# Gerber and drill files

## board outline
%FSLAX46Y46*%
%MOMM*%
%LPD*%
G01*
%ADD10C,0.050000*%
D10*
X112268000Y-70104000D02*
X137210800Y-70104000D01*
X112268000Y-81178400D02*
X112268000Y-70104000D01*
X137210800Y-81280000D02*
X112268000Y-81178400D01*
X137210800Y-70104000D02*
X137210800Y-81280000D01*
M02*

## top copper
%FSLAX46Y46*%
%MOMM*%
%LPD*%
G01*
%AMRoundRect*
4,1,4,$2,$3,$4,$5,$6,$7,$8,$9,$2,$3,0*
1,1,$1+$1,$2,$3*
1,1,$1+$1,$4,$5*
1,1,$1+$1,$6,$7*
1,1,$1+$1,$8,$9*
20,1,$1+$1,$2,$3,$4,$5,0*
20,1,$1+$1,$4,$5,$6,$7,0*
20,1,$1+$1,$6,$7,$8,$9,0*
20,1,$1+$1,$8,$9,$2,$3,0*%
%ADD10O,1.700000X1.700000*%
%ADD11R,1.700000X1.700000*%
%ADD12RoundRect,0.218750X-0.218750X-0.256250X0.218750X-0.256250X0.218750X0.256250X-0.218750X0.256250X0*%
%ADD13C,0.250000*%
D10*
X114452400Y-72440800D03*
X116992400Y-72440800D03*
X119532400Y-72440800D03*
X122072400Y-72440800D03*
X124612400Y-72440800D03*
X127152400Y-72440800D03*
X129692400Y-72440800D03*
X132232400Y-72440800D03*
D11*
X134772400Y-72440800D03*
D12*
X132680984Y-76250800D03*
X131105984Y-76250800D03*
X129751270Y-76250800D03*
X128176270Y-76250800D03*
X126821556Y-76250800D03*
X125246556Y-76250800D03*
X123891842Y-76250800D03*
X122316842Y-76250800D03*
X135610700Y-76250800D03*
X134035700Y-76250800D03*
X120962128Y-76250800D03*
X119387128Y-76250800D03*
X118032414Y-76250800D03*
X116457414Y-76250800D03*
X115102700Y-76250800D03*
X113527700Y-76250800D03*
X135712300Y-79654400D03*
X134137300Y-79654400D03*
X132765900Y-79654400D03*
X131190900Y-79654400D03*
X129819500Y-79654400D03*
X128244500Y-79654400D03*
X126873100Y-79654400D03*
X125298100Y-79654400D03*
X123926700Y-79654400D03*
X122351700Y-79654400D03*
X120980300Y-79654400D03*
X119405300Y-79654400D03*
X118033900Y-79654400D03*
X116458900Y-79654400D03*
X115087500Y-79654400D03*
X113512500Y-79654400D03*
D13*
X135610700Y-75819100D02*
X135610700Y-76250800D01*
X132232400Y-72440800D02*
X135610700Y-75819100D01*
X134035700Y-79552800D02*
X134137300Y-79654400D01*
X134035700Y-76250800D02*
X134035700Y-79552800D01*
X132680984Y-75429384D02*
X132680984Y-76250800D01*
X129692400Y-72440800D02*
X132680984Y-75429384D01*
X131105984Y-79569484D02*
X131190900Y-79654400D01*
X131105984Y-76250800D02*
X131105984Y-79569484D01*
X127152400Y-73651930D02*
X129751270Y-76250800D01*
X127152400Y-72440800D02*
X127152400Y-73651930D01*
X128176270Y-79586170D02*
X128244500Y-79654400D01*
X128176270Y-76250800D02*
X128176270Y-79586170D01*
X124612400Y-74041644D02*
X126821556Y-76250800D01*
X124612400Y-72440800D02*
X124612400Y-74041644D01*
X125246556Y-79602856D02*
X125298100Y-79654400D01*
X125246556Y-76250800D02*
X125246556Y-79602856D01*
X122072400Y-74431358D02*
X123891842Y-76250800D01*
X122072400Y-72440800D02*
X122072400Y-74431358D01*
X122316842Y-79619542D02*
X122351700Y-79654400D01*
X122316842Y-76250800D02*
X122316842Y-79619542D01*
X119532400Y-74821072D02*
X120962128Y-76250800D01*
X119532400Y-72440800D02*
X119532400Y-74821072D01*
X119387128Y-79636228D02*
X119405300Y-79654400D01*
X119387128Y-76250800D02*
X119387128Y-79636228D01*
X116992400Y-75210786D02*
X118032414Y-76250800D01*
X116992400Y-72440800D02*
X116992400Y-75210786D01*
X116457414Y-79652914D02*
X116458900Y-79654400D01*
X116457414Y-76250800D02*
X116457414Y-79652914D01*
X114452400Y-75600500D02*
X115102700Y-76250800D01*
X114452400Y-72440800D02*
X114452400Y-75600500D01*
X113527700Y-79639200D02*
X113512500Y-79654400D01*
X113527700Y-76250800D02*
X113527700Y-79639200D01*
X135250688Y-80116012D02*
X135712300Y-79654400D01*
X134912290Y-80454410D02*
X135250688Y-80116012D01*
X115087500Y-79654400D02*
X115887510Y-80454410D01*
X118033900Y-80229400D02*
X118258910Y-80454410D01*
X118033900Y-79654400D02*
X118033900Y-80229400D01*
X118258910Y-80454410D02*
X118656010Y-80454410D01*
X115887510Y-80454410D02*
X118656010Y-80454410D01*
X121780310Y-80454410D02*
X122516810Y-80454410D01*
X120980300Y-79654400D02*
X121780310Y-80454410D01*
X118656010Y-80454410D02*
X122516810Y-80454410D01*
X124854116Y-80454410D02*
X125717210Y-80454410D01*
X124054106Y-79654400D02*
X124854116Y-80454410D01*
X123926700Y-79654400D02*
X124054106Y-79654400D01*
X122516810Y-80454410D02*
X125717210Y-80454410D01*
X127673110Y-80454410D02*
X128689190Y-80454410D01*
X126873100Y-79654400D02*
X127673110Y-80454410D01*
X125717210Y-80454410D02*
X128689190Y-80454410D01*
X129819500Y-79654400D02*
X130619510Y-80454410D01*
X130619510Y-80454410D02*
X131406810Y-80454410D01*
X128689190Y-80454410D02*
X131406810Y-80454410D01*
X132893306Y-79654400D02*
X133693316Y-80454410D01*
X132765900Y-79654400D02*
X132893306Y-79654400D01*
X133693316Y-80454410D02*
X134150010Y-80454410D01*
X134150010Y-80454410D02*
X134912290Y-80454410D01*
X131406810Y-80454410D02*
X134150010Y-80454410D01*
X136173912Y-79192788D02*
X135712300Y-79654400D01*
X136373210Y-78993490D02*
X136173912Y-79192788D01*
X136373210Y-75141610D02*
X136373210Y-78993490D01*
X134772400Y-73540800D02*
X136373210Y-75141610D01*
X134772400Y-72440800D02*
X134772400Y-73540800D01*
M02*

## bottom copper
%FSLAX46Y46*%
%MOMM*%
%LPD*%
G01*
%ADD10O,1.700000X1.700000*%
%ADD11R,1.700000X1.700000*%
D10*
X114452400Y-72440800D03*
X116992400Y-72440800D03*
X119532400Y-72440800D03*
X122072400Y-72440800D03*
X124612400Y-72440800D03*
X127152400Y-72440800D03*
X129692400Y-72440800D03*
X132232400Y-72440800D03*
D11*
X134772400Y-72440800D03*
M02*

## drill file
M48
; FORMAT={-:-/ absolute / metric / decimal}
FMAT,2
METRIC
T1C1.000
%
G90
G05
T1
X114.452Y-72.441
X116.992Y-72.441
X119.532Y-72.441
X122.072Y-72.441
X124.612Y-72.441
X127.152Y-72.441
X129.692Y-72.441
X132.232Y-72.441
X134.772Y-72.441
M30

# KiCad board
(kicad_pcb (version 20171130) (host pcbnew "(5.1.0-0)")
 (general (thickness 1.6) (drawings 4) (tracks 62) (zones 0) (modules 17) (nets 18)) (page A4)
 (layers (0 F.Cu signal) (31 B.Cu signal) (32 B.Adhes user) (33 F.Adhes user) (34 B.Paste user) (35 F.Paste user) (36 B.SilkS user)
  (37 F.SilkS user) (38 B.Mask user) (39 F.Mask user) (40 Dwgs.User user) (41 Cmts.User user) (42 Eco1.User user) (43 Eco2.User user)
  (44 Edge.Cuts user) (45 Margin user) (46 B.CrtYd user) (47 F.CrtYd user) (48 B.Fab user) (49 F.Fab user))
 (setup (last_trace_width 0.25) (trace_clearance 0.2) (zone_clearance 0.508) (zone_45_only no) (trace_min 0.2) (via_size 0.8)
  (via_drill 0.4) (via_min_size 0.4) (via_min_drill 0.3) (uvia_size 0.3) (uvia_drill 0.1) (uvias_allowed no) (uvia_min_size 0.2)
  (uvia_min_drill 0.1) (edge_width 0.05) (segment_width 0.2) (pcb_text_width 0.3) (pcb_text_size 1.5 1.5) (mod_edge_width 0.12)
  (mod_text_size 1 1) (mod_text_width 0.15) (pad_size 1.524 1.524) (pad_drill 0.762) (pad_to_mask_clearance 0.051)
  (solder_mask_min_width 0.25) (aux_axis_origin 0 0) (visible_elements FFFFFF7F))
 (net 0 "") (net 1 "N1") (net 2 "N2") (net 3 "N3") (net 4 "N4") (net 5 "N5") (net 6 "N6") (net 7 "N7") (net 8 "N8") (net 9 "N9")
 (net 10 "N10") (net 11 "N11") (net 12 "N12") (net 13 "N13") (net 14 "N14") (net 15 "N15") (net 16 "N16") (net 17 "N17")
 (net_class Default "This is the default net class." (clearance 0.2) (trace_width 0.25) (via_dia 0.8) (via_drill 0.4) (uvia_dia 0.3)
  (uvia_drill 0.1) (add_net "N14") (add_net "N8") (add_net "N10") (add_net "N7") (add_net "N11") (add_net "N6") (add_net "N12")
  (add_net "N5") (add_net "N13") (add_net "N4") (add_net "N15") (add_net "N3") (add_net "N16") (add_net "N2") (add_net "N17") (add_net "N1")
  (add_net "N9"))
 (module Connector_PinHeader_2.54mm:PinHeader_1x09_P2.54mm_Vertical (layer B.Cu) (at 134.7724 72.4408 90)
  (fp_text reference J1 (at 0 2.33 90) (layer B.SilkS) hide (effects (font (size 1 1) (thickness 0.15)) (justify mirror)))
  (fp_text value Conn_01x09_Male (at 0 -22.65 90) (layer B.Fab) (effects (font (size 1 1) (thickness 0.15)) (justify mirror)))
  (pad 9 thru_hole oval (at 0 -20.32 90) (size 1.7 1.7) (drill 1) (layers *.Cu *.Mask) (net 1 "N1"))
  (pad 8 thru_hole oval (at 0 -17.78 90) (size 1.7 1.7) (drill 1) (layers *.Cu *.Mask) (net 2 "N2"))
  (pad 7 thru_hole oval (at 0 -15.24 90) (size 1.7 1.7) (drill 1) (layers *.Cu *.Mask) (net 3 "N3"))
  (pad 6 thru_hole oval (at 0 -12.7 90) (size 1.7 1.7) (drill 1) (layers *.Cu *.Mask) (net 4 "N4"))
  (pad 5 thru_hole oval (at 0 -10.16 90) (size 1.7 1.7) (drill 1) (layers *.Cu *.Mask) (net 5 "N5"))
  (pad 4 thru_hole oval (at 0 -7.62 90) (size 1.7 1.7) (drill 1) (layers *.Cu *.Mask) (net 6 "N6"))
  (pad 3 thru_hole oval (at 0 -5.08 90) (size 1.7 1.7) (drill 1) (layers *.Cu *.Mask) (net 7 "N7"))
  (pad 2 thru_hole oval (at 0 -2.54 90) (size 1.7 1.7) (drill 1) (layers *.Cu *.Mask) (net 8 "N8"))
  (pad 1 thru_hole rect (at 0 0 90) (size 1.7 1.7) (drill 1) (layers *.Cu *.Mask) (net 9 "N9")))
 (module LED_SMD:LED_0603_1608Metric (layer F.Cu) (at 131.893484 76.2508)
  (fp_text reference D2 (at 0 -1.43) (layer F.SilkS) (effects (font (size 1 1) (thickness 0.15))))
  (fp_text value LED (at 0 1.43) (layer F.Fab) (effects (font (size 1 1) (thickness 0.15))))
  (pad 2 smd roundrect (at 0.7875 0) (size 0.875 0.95) (layers F.Cu F.Paste F.Mask) (roundrect_rratio 0.25) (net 7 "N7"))
  (pad 1 smd roundrect (at -0.7875 0) (size 0.875 0.95) (layers F.Cu F.Paste F.Mask) (roundrect_rratio 0.25) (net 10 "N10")))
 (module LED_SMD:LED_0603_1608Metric (layer F.Cu) (at 128.96377 76.2508)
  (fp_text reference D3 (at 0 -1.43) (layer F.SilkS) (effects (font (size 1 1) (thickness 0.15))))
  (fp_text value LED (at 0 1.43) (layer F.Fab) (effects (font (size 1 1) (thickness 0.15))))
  (pad 2 smd roundrect (at 0.7875 0) (size 0.875 0.95) (layers F.Cu F.Paste F.Mask) (roundrect_rratio 0.25) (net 6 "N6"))
  (pad 1 smd roundrect (at -0.7875 0) (size 0.875 0.95) (layers F.Cu F.Paste F.Mask) (roundrect_rratio 0.25) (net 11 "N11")))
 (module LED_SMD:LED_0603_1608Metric (layer F.Cu) (at 126.034056 76.2508)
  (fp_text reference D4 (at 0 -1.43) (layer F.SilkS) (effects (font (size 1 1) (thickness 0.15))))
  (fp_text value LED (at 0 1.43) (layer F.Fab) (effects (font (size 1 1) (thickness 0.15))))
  (pad 2 smd roundrect (at 0.7875 0) (size 0.875 0.95) (layers F.Cu F.Paste F.Mask) (roundrect_rratio 0.25) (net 5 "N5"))
  (pad 1 smd roundrect (at -0.7875 0) (size 0.875 0.95) (layers F.Cu F.Paste F.Mask) (roundrect_rratio 0.25) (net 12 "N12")))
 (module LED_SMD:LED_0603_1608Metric (layer F.Cu) (at 123.104342 76.2508)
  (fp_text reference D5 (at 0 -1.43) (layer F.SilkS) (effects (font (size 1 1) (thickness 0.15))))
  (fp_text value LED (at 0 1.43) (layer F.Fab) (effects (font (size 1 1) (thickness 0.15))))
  (pad 2 smd roundrect (at 0.7875 0) (size 0.875 0.95) (layers F.Cu F.Paste F.Mask) (roundrect_rratio 0.25) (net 4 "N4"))
  (pad 1 smd roundrect (at -0.7875 0) (size 0.875 0.95) (layers F.Cu F.Paste F.Mask) (roundrect_rratio 0.25) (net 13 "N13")))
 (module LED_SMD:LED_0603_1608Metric (layer F.Cu) (at 134.8232 76.2508)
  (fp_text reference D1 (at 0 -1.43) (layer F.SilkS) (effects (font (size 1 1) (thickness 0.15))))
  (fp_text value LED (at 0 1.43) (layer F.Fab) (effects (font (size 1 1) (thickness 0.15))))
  (pad 2 smd roundrect (at 0.7875 0) (size 0.875 0.95) (layers F.Cu F.Paste F.Mask) (roundrect_rratio 0.25) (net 8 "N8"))
  (pad 1 smd roundrect (at -0.7875 0) (size 0.875 0.95) (layers F.Cu F.Paste F.Mask) (roundrect_rratio 0.25) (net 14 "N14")))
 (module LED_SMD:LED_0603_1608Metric (layer F.Cu) (at 120.174628 76.2508)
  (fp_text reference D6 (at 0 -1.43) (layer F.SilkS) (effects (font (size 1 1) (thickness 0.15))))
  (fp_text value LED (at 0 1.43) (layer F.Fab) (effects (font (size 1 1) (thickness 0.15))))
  (pad 2 smd roundrect (at 0.7875 0) (size 0.875 0.95) (layers F.Cu F.Paste F.Mask) (roundrect_rratio 0.25) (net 3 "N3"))
  (pad 1 smd roundrect (at -0.7875 0) (size 0.875 0.95) (layers F.Cu F.Paste F.Mask) (roundrect_rratio 0.25) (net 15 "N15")))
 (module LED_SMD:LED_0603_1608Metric (layer F.Cu) (at 117.244914 76.2508)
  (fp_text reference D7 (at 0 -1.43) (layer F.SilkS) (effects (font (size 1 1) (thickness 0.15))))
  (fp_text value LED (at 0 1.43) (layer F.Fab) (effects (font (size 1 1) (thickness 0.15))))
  (pad 2 smd roundrect (at 0.7875 0) (size 0.875 0.95) (layers F.Cu F.Paste F.Mask) (roundrect_rratio 0.25) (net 2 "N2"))
  (pad 1 smd roundrect (at -0.7875 0) (size 0.875 0.95) (layers F.Cu F.Paste F.Mask) (roundrect_rratio 0.25) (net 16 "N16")))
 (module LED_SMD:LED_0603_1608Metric (layer F.Cu) (at 114.3152 76.2508)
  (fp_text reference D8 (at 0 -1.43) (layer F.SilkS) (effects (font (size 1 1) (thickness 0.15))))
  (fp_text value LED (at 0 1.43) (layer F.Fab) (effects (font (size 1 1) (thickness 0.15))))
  (pad 2 smd roundrect (at 0.7875 0) (size 0.875 0.95) (layers F.Cu F.Paste F.Mask) (roundrect_rratio 0.25) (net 1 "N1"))
  (pad 1 smd roundrect (at -0.7875 0) (size 0.875 0.95) (layers F.Cu F.Paste F.Mask) (roundrect_rratio 0.25) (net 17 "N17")))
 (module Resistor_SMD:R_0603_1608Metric (layer F.Cu) (at 134.9248 79.6544)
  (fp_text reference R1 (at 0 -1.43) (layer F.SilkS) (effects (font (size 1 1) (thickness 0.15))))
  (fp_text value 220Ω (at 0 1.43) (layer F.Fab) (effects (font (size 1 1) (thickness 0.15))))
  (pad 2 smd roundrect (at 0.7875 0) (size 0.875 0.95) (layers F.Cu F.Paste F.Mask) (roundrect_rratio 0.25) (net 9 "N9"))
  (pad 1 smd roundrect (at -0.7875 0) (size 0.875 0.95) (layers F.Cu F.Paste F.Mask) (roundrect_rratio 0.25) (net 14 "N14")))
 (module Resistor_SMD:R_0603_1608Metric (layer F.Cu) (at 131.9784 79.6544)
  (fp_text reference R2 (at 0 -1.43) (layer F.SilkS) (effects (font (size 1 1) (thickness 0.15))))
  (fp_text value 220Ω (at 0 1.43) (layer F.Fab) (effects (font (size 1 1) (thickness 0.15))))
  (pad 2 smd roundrect (at 0.7875 0) (size 0.875 0.95) (layers F.Cu F.Paste F.Mask) (roundrect_rratio 0.25) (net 9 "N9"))
  (pad 1 smd roundrect (at -0.7875 0) (size 0.875 0.95) (layers F.Cu F.Paste F.Mask) (roundrect_rratio 0.25) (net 10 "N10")))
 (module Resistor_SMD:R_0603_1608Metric (layer F.Cu) (at 129.032 79.6544)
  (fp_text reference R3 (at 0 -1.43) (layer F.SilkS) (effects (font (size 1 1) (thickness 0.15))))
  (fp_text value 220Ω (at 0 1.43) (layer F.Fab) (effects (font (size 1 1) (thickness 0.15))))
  (pad 2 smd roundrect (at 0.7875 0) (size 0.875 0.95) (layers F.Cu F.Paste F.Mask) (roundrect_rratio 0.25) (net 9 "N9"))
  (pad 1 smd roundrect (at -0.7875 0) (size 0.875 0.95) (layers F.Cu F.Paste F.Mask) (roundrect_rratio 0.25) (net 11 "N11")))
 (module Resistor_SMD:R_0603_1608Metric (layer F.Cu) (at 126.0856 79.6544)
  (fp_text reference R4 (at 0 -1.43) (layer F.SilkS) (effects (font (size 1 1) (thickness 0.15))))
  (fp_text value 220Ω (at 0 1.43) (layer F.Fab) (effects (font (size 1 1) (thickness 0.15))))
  (pad 2 smd roundrect (at 0.7875 0) (size 0.875 0.95) (layers F.Cu F.Paste F.Mask) (roundrect_rratio 0.25) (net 9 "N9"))
  (pad 1 smd roundrect (at -0.7875 0) (size 0.875 0.95) (layers F.Cu F.Paste F.Mask) (roundrect_rratio 0.25) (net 12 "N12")))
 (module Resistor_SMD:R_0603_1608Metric (layer F.Cu) (at 123.1392 79.6544)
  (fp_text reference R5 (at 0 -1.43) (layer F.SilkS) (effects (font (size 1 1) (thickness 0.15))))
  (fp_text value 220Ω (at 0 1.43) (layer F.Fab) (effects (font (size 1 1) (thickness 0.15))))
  (pad 2 smd roundrect (at 0.7875 0) (size 0.875 0.95) (layers F.Cu F.Paste F.Mask) (roundrect_rratio 0.25) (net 9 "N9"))
  (pad 1 smd roundrect (at -0.7875 0) (size 0.875 0.95) (layers F.Cu F.Paste F.Mask) (roundrect_rratio 0.25) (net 13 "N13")))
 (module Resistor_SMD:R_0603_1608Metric (layer F.Cu) (at 120.1928 79.6544)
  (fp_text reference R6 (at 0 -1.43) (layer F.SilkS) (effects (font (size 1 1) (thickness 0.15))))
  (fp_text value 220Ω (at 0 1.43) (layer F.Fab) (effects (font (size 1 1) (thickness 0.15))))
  (pad 2 smd roundrect (at 0.7875 0) (size 0.875 0.95) (layers F.Cu F.Paste F.Mask) (roundrect_rratio 0.25) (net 9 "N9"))
  (pad 1 smd roundrect (at -0.7875 0) (size 0.875 0.95) (layers F.Cu F.Paste F.Mask) (roundrect_rratio 0.25) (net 15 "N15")))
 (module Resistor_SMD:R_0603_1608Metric (layer F.Cu) (at 117.2464 79.6544)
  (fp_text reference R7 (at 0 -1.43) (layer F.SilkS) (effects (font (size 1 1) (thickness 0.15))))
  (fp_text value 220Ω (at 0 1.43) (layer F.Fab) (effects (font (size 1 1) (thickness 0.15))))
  (pad 2 smd roundrect (at 0.7875 0) (size 0.875 0.95) (layers F.Cu F.Paste F.Mask) (roundrect_rratio 0.25) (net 9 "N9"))
  (pad 1 smd roundrect (at -0.7875 0) (size 0.875 0.95) (layers F.Cu F.Paste F.Mask) (roundrect_rratio 0.25) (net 16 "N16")))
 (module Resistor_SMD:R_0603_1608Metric (layer F.Cu) (at 114.3 79.6544)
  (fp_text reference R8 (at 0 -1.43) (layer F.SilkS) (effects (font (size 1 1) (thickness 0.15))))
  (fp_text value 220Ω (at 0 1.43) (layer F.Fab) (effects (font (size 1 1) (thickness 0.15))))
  (pad 2 smd roundrect (at 0.7875 0) (size 0.875 0.95) (layers F.Cu F.Paste F.Mask) (roundrect_rratio 0.25) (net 9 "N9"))
  (pad 1 smd roundrect (at -0.7875 0) (size 0.875 0.95) (layers F.Cu F.Paste F.Mask) (roundrect_rratio 0.25) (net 17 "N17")))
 (gr_line (start 112.268 70.104) (end 137.2108 70.104) (layer Edge.Cuts) (width 0.05))
 (gr_line (start 112.268 81.1784) (end 112.268 70.104) (layer Edge.Cuts) (width 0.05))
 (gr_line (start 137.2108 81.28) (end 112.268 81.1784) (layer Edge.Cuts) (width 0.05))
 (gr_line (start 137.2108 70.104) (end 137.2108 81.28) (layer Edge.Cuts) (width 0.05))
 (segment (start 135.6107 75.8191) (end 135.6107 76.2508) (width 0.25) (layer F.Cu) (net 8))
 (segment (start 132.2324 72.4408) (end 135.6107 75.8191) (width 0.25) (layer F.Cu) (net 8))
 (segment (start 134.0357 79.5528) (end 134.1373 79.6544) (width 0.25) (layer F.Cu) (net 14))
 (segment (start 134.0357 76.2508) (end 134.0357 79.5528) (width 0.25) (layer F.Cu) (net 14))
 (segment (start 132.680984 75.429384) (end 132.680984 76.2508) (width 0.25) (layer F.Cu) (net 7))
 (segment (start 129.6924 72.4408) (end 132.680984 75.429384) (width 0.25) (layer F.Cu) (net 7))
 (segment (start 131.105984 79.569484) (end 131.1909 79.6544) (width 0.25) (layer F.Cu) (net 10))
 (segment (start 131.105984 76.2508) (end 131.105984 79.569484) (width 0.25) (layer F.Cu) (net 10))
 (segment (start 127.1524 73.65193) (end 129.75127 76.2508) (width 0.25) (layer F.Cu) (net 6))
 (segment (start 127.1524 72.4408) (end 127.1524 73.65193) (width 0.25) (layer F.Cu) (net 6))
 (segment (start 128.17627 79.58617) (end 128.2445 79.6544) (width 0.25) (layer F.Cu) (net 11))
 (segment (start 128.17627 76.2508) (end 128.17627 79.58617) (width 0.25) (layer F.Cu) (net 11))
 (segment (start 124.6124 74.041644) (end 126.821556 76.2508) (width 0.25) (layer F.Cu) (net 5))
 (segment (start 124.6124 72.4408) (end 124.6124 74.041644) (width 0.25) (layer F.Cu) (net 5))
 (segment (start 125.246556 79.602856) (end 125.2981 79.6544) (width 0.25) (layer F.Cu) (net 12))
 (segment (start 125.246556 76.2508) (end 125.246556 79.602856) (width 0.25) (layer F.Cu) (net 12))
 (segment (start 122.0724 74.431358) (end 123.891842 76.2508) (width 0.25) (layer F.Cu) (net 4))
 (segment (start 122.0724 72.4408) (end 122.0724 74.431358) (width 0.25) (layer F.Cu) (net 4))
 (segment (start 122.316842 79.619542) (end 122.3517 79.6544) (width 0.25) (layer F.Cu) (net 13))
 (segment (start 122.316842 76.2508) (end 122.316842 79.619542) (width 0.25) (layer F.Cu) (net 13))
 (segment (start 119.5324 74.821072) (end 120.962128 76.2508) (width 0.25) (layer F.Cu) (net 3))
 (segment (start 119.5324 72.4408) (end 119.5324 74.821072) (width 0.25) (layer F.Cu) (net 3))
 (segment (start 119.387128 79.636228) (end 119.4053 79.6544) (width 0.25) (layer F.Cu) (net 15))
 (segment (start 119.387128 76.2508) (end 119.387128 79.636228) (width 0.25) (layer F.Cu) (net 15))
 (segment (start 116.9924 75.210786) (end 118.032414 76.2508) (width 0.25) (layer F.Cu) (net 2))
 (segment (start 116.9924 72.4408) (end 116.9924 75.210786) (width 0.25) (layer F.Cu) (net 2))
 (segment (start 116.457414 79.652914) (end 116.4589 79.6544) (width 0.25) (layer F.Cu) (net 16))
 (segment (start 116.457414 76.2508) (end 116.457414 79.652914) (width 0.25) (layer F.Cu) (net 16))
 (segment (start 114.4524 75.6005) (end 115.1027 76.2508) (width 0.25) (layer F.Cu) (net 1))
 (segment (start 114.4524 72.4408) (end 114.4524 75.6005) (width 0.25) (layer F.Cu) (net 1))
 (segment (start 113.5277 79.6392) (end 113.5125 79.6544) (width 0.25) (layer F.Cu) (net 17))
 (segment (start 113.5277 76.2508) (end 113.5277 79.6392) (width 0.25) (layer F.Cu) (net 17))
 (segment (start 135.250688 80.116012) (end 135.7123 79.6544) (width 0.25) (layer F.Cu) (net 9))
 (segment (start 134.91229 80.45441) (end 135.250688 80.116012) (width 0.25) (layer F.Cu) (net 9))
 (segment (start 115.0875 79.6544) (end 115.88751 80.45441) (width 0.25) (layer F.Cu) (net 9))
 (segment (start 118.0339 80.2294) (end 118.25891 80.45441) (width 0.25) (layer F.Cu) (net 9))
 (segment (start 118.0339 79.6544) (end 118.0339 80.2294) (width 0.25) (layer F.Cu) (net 9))
 (segment (start 118.25891 80.45441) (end 118.65601 80.45441) (width 0.25) (layer F.Cu) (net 9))
 (segment (start 115.88751 80.45441) (end 118.65601 80.45441) (width 0.25) (layer F.Cu) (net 9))
 (segment (start 121.78031 80.45441) (end 122.51681 80.45441) (width 0.25) (layer F.Cu) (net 9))
 (segment (start 120.9803 79.6544) (end 121.78031 80.45441) (width 0.25) (layer F.Cu) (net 9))
 (segment (start 118.65601 80.45441) (end 122.51681 80.45441) (width 0.25) (layer F.Cu) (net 9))
 (segment (start 124.854116 80.45441) (end 125.71721 80.45441) (width 0.25) (layer F.Cu) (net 9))
 (segment (start 124.054106 79.6544) (end 124.854116 80.45441) (width 0.25) (layer F.Cu) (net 9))
 (segment (start 123.9267 79.6544) (end 124.054106 79.6544) (width 0.25) (layer F.Cu) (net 9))
 (segment (start 122.51681 80.45441) (end 125.71721 80.45441) (width 0.25) (layer F.Cu) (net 9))
 (segment (start 127.67311 80.45441) (end 128.68919 80.45441) (width 0.25) (layer F.Cu) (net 9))
 (segment (start 126.8731 79.6544) (end 127.67311 80.45441) (width 0.25) (layer F.Cu) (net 9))
 (segment (start 125.71721 80.45441) (end 128.68919 80.45441) (width 0.25) (layer F.Cu) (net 9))
 (segment (start 129.8195 79.6544) (end 130.61951 80.45441) (width 0.25) (layer F.Cu) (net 9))
 (segment (start 130.61951 80.45441) (end 131.40681 80.45441) (width 0.25) (layer F.Cu) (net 9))
 (segment (start 128.68919 80.45441) (end 131.40681 80.45441) (width 0.25) (layer F.Cu) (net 9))
 (segment (start 132.893306 79.6544) (end 133.693316 80.45441) (width 0.25) (layer F.Cu) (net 9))
 (segment (start 132.7659 79.6544) (end 132.893306 79.6544) (width 0.25) (layer F.Cu) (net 9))
 (segment (start 133.693316 80.45441) (end 134.15001 80.45441) (width 0.25) (layer F.Cu) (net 9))
 (segment (start 134.15001 80.45441) (end 134.91229 80.45441) (width 0.25) (layer F.Cu) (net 9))
 (segment (start 131.40681 80.45441) (end 134.15001 80.45441) (width 0.25) (layer F.Cu) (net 9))
 (segment (start 136.173912 79.192788) (end 135.7123 79.6544) (width 0.25) (layer F.Cu) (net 9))
 (segment (start 136.37321 78.99349) (end 136.173912 79.192788) (width 0.25) (layer F.Cu) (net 9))
 (segment (start 136.37321 75.14161) (end 136.37321 78.99349) (width 0.25) (layer F.Cu) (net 9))
 (segment (start 134.7724 73.5408) (end 136.37321 75.14161) (width 0.25) (layer F.Cu) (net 9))
 (segment (start 134.7724 72.4408) (end 134.7724 73.5408) (width 0.25) (layer F.Cu) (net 9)))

